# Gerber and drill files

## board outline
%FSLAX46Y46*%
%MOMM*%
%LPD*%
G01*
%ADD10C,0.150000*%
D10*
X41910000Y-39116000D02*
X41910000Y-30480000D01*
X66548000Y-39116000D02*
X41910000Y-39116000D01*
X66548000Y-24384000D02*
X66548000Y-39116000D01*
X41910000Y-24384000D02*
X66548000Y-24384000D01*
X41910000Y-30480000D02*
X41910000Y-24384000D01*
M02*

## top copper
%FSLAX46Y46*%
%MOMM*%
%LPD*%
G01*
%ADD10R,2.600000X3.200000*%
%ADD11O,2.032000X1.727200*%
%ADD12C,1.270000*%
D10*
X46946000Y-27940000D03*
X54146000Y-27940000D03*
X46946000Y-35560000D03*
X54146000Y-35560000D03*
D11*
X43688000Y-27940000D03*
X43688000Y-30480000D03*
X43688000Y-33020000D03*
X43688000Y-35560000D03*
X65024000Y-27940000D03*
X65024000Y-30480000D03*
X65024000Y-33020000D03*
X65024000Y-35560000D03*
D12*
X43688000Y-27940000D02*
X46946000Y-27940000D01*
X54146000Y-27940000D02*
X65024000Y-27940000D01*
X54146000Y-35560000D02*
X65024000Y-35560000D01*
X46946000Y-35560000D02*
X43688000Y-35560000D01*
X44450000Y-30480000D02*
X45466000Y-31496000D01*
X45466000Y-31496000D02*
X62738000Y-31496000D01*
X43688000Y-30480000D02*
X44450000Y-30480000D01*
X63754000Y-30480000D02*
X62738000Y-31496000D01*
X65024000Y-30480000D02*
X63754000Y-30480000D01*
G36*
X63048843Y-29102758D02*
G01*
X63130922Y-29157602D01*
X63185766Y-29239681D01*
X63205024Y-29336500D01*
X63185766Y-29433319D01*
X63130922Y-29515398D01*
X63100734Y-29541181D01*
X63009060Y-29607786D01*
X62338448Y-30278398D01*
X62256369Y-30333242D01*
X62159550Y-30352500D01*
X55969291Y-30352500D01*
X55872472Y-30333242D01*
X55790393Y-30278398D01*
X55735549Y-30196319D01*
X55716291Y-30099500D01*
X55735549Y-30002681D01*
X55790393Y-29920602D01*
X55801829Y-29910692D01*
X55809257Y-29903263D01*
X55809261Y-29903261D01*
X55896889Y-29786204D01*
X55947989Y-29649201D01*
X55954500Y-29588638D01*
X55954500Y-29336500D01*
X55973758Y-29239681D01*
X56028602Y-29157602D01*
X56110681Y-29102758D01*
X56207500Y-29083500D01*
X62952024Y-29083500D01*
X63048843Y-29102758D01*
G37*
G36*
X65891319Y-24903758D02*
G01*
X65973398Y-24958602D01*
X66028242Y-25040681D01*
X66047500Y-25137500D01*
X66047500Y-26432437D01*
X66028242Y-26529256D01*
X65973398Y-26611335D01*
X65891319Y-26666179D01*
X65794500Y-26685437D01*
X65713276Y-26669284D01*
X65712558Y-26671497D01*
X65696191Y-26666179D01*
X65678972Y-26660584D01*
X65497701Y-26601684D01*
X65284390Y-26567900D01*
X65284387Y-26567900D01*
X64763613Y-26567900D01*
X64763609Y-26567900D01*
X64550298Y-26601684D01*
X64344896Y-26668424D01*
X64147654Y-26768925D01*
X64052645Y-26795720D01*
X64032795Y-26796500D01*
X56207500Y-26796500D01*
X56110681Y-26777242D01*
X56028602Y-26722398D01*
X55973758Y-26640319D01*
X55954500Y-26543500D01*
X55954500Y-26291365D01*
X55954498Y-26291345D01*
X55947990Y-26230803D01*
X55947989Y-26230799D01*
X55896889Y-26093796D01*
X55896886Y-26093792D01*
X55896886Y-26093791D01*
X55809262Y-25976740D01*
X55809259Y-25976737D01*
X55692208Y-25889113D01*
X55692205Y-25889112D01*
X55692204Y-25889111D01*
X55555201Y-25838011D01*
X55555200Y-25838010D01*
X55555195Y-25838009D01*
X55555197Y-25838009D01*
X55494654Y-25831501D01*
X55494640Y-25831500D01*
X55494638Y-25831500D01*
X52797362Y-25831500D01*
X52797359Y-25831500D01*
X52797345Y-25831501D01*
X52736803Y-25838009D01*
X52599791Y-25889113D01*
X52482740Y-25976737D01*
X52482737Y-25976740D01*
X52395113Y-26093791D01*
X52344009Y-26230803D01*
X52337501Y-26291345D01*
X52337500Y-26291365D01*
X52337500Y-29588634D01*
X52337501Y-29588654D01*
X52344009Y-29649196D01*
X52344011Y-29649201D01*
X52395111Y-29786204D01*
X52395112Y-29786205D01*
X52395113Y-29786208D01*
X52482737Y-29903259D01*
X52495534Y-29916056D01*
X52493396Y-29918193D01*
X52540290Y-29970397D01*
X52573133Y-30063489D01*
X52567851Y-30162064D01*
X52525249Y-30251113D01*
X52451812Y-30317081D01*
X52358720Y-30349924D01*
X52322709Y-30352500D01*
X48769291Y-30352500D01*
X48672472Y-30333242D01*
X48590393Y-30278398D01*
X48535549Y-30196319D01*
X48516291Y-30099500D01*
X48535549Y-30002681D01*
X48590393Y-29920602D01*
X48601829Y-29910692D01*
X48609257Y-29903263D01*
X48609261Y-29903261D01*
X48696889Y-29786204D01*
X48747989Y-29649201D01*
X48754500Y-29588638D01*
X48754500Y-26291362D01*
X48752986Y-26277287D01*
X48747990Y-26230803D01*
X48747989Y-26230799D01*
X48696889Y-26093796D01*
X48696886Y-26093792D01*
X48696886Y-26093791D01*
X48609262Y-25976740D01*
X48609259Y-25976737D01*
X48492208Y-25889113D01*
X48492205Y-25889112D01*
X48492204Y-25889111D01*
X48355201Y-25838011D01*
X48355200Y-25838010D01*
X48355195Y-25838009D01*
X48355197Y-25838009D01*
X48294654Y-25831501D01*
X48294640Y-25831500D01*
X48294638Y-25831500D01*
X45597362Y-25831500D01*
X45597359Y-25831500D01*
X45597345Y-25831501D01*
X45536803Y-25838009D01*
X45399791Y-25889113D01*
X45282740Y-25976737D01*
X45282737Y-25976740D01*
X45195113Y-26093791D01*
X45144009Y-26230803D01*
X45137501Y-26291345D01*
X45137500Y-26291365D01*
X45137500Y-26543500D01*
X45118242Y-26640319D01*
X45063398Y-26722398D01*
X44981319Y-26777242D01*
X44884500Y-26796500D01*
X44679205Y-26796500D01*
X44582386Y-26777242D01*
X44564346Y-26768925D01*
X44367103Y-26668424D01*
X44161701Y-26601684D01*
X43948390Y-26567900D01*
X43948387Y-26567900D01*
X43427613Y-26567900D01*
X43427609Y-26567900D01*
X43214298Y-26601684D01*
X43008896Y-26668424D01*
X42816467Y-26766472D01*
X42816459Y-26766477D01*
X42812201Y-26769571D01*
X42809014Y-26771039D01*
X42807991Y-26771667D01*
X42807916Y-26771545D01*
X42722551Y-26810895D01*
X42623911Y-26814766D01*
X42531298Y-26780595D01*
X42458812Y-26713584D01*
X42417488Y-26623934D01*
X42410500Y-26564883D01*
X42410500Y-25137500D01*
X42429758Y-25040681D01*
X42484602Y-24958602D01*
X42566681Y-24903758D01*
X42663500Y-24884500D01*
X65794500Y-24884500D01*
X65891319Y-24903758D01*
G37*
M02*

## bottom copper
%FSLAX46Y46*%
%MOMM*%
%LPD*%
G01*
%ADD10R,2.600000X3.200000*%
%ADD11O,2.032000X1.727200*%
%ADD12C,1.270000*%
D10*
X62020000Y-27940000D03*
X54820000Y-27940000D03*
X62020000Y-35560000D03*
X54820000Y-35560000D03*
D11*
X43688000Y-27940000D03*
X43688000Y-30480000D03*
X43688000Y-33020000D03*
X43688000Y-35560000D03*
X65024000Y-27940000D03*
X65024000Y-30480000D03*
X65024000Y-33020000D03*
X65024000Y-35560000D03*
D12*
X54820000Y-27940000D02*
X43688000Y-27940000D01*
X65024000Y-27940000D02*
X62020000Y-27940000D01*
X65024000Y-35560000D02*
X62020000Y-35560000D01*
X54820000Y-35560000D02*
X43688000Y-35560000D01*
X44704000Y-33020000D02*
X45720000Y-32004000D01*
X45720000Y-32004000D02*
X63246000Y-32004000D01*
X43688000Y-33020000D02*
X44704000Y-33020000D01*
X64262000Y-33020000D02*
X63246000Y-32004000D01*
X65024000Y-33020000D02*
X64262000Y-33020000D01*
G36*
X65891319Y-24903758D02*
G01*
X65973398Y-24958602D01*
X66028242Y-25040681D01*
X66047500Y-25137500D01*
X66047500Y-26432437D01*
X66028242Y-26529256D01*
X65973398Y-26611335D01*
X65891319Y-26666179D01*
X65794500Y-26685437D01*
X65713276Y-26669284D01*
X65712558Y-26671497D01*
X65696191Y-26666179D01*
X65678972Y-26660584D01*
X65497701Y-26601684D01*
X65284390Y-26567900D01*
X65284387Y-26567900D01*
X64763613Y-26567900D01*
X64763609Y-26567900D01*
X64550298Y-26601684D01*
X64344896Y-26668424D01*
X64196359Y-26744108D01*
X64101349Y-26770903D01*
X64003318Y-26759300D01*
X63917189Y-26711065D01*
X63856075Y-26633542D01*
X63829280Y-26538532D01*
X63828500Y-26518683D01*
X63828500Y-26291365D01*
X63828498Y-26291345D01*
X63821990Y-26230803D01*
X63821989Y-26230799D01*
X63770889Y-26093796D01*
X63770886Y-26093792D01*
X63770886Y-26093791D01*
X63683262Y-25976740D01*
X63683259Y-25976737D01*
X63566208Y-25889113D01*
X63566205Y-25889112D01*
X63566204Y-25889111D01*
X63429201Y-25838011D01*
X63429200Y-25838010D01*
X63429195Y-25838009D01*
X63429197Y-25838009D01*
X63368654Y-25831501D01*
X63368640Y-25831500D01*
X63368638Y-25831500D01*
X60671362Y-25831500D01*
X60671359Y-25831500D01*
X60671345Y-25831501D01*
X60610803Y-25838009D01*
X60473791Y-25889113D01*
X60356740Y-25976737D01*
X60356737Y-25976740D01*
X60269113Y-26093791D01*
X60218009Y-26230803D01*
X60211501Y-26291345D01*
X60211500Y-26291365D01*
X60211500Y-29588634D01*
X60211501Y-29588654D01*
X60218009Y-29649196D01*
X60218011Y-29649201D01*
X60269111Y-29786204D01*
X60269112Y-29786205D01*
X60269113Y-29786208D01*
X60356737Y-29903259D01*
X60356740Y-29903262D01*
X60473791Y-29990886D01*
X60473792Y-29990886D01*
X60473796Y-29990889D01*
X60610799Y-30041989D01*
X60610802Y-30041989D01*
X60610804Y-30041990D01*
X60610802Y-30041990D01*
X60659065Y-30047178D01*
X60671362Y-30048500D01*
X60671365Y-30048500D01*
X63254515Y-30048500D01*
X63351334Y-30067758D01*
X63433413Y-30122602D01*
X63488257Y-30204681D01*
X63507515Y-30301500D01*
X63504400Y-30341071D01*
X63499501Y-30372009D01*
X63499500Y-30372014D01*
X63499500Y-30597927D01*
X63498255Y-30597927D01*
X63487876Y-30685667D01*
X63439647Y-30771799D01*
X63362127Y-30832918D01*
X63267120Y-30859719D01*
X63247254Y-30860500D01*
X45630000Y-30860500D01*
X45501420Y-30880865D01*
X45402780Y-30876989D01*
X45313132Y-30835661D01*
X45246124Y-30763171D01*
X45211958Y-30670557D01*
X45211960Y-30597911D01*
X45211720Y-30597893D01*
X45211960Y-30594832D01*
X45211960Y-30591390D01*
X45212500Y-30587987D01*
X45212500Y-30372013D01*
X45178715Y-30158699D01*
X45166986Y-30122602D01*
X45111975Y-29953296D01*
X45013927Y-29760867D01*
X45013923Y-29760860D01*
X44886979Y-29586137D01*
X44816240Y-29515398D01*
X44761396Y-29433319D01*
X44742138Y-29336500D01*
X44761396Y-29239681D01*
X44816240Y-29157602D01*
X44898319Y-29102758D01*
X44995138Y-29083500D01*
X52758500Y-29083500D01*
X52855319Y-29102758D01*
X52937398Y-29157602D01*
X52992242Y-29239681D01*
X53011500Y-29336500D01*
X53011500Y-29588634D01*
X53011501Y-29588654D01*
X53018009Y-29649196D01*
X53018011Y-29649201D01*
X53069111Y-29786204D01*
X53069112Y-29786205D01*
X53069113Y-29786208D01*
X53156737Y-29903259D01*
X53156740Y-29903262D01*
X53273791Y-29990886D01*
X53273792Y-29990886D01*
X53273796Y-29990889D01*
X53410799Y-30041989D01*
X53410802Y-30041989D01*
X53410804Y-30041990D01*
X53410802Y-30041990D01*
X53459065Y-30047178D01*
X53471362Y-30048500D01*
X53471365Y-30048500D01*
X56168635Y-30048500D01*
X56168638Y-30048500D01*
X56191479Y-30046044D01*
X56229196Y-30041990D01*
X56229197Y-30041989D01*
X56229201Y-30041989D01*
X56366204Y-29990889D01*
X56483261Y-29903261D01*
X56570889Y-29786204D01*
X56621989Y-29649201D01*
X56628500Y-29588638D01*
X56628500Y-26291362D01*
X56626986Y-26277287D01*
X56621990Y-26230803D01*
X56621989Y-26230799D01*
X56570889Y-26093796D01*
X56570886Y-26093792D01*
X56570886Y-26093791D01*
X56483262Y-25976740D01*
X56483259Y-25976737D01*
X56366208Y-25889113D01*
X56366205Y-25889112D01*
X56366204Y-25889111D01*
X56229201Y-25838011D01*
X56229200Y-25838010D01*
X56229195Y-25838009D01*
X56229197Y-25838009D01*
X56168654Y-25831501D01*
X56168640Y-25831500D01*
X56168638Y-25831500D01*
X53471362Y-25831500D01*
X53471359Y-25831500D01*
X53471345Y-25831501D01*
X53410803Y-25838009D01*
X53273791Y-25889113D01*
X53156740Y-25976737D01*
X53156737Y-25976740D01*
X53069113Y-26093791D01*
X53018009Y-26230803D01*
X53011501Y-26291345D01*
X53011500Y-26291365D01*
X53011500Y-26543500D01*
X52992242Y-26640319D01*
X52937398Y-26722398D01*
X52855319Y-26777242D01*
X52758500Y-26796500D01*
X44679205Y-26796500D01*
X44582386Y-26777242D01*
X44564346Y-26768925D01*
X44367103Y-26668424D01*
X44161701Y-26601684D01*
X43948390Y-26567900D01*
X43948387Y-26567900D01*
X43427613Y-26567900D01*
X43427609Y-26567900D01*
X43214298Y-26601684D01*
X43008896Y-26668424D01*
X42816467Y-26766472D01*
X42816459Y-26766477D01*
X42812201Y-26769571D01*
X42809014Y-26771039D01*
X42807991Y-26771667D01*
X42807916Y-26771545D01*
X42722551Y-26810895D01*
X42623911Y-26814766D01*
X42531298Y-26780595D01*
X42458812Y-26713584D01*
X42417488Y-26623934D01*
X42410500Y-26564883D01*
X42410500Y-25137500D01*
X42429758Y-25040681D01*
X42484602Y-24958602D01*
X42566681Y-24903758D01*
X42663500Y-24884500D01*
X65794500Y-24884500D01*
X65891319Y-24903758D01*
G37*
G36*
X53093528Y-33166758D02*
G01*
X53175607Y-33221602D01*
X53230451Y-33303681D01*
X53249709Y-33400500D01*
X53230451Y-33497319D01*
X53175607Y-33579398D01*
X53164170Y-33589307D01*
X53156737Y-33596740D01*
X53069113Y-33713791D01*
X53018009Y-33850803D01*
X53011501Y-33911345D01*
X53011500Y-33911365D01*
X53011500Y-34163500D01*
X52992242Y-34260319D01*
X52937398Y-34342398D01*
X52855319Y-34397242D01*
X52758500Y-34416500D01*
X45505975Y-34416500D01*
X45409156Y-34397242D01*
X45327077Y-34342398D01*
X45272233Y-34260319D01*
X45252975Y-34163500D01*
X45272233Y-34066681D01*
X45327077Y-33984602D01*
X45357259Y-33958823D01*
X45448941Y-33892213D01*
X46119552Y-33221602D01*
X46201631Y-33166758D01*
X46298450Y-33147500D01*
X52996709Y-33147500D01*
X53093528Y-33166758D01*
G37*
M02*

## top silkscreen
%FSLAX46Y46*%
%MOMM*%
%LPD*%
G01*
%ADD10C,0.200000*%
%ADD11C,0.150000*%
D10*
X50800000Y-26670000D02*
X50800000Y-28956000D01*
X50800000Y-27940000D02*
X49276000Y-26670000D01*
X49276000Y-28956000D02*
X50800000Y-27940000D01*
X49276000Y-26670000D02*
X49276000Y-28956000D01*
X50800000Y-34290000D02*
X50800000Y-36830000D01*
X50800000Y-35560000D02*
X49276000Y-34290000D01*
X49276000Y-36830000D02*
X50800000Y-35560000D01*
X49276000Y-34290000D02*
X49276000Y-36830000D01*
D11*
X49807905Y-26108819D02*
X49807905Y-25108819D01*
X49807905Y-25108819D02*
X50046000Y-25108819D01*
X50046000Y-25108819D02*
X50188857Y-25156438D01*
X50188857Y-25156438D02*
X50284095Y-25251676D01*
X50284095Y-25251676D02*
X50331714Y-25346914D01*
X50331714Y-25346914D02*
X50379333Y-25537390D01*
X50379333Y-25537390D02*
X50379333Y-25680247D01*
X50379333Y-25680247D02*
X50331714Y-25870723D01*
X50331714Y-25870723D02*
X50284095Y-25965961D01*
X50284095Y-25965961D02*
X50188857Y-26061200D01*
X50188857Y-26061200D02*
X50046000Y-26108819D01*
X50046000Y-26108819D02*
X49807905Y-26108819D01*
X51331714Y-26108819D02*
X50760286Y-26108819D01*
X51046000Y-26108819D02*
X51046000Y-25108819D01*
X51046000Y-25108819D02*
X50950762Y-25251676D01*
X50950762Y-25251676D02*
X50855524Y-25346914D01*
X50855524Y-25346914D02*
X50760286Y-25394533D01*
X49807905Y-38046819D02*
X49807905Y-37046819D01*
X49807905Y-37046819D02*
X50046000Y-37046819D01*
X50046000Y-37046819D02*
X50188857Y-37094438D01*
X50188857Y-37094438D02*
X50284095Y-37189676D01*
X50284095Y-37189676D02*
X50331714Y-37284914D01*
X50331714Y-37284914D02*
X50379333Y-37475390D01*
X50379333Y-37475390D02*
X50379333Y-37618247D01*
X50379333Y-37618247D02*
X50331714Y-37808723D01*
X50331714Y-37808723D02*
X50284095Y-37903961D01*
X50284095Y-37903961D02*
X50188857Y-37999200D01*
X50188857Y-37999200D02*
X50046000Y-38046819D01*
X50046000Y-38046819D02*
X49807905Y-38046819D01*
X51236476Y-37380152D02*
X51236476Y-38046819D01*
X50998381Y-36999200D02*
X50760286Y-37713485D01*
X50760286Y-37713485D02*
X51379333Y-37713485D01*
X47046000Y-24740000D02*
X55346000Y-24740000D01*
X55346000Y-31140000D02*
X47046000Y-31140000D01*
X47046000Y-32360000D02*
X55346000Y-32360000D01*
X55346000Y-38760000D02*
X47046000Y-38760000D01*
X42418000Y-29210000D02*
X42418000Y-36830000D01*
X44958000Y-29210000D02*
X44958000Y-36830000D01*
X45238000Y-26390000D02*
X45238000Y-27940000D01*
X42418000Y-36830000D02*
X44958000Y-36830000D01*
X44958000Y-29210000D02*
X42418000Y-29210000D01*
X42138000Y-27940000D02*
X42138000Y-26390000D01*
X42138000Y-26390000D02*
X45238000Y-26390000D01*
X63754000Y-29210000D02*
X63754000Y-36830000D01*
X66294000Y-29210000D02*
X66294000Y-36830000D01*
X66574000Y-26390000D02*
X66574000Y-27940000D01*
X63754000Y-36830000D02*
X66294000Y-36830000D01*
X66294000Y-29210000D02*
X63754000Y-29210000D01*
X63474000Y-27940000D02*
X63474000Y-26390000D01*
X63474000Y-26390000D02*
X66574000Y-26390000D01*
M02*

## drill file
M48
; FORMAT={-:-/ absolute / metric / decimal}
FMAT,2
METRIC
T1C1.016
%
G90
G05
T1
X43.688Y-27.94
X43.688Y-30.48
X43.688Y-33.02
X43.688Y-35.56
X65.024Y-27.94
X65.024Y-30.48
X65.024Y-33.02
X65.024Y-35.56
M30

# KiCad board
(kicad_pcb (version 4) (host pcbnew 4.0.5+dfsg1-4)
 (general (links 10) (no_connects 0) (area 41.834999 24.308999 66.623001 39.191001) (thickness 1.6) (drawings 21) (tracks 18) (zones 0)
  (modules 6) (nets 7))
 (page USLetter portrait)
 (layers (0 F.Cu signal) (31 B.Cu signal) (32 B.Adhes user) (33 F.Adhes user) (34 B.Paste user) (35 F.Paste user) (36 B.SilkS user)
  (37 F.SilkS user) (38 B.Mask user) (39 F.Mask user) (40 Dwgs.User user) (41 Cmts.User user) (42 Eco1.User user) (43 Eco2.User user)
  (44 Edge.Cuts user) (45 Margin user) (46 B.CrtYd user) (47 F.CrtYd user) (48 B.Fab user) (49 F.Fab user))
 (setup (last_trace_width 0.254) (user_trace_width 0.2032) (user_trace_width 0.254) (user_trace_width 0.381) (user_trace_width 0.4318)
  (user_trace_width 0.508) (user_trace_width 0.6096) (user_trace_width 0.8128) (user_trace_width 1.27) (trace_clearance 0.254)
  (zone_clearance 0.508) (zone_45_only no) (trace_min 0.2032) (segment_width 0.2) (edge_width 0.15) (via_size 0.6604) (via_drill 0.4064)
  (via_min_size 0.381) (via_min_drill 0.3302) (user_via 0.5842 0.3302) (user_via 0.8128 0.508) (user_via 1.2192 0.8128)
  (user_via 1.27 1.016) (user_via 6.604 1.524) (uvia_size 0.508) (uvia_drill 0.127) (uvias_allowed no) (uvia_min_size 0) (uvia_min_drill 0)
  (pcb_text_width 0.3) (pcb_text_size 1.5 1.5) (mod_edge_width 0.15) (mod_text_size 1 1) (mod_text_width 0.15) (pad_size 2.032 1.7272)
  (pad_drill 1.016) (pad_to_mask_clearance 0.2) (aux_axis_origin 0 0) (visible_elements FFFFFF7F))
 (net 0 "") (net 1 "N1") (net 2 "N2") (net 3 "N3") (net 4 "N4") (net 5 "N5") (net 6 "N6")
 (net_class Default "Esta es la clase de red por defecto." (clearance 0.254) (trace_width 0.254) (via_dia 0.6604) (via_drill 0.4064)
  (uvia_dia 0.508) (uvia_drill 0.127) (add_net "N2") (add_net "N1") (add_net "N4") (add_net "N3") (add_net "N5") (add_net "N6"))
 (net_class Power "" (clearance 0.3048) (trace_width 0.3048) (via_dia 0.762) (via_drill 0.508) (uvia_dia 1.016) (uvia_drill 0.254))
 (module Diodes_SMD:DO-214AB (layer F.Cu) (at 50.546 27.94 180)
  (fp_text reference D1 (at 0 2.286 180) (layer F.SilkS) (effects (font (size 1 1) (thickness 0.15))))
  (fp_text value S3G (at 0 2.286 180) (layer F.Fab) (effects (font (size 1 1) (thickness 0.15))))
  (fp_line (start 3.5 3.2) (end -4.8 3.2) (layer F.SilkS) (width 0.15))
  (fp_line (start -4.8 -3.2) (end 3.5 -3.2) (layer F.SilkS) (width 0.15))
  (pad 2 smd rect (at 3.6 0 180) (size 2.6 3.2) (layers F.Cu F.Paste F.Mask) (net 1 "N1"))
  (pad 1 smd rect (at -3.6 0 180) (size 2.6 3.2) (layers F.Cu F.Paste F.Mask) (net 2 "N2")))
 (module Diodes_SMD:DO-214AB (layer B.Cu) (at 58.42 27.94)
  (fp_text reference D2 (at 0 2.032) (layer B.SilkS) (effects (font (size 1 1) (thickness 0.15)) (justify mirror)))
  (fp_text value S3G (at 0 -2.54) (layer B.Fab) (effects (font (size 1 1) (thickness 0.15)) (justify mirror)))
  (pad 2 smd rect (at 3.6 0) (size 2.6 3.2) (layers B.Cu B.Paste B.Mask) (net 2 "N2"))
  (pad 1 smd rect (at -3.6 0) (size 2.6 3.2) (layers B.Cu B.Paste B.Mask) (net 1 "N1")))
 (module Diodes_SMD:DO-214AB (layer B.Cu) (at 58.42 35.56)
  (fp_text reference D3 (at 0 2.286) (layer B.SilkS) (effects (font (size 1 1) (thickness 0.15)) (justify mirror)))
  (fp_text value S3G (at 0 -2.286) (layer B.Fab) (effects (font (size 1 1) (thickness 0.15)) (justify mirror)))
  (pad 2 smd rect (at 3.6 0) (size 2.6 3.2) (layers B.Cu B.Paste B.Mask) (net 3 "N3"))
  (pad 1 smd rect (at -3.6 0) (size 2.6 3.2) (layers B.Cu B.Paste B.Mask) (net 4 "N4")))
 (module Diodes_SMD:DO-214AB (layer F.Cu) (at 50.546 35.56 180)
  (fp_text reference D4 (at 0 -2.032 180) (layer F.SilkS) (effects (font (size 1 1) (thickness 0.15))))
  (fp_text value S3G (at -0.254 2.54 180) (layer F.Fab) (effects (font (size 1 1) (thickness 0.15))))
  (fp_line (start 3.5 3.2) (end -4.8 3.2) (layer F.SilkS) (width 0.15))
  (fp_line (start -4.8 -3.2) (end 3.5 -3.2) (layer F.SilkS) (width 0.15))
  (pad 2 smd rect (at 3.6 0 180) (size 2.6 3.2) (layers F.Cu F.Paste F.Mask) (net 4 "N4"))
  (pad 1 smd rect (at -3.6 0 180) (size 2.6 3.2) (layers F.Cu F.Paste F.Mask) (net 3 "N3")))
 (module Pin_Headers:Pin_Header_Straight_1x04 (layer F.Cu) (at 43.688 27.94)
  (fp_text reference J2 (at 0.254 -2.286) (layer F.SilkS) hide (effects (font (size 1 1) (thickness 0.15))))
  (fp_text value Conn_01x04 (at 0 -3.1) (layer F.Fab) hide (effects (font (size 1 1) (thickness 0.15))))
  (fp_line (start -1.27 1.27) (end -1.27 8.89) (layer F.SilkS) (width 0.15))
  (fp_line (start 1.27 1.27) (end 1.27 8.89) (layer F.SilkS) (width 0.15))
  (fp_line (start 1.55 -1.55) (end 1.55 0) (layer F.SilkS) (width 0.15))
  (fp_line (start -1.27 8.89) (end 1.27 8.89) (layer F.SilkS) (width 0.15))
  (fp_line (start 1.27 1.27) (end -1.27 1.27) (layer F.SilkS) (width 0.15))
  (fp_line (start -1.55 0) (end -1.55 -1.55) (layer F.SilkS) (width 0.15))
  (fp_line (start -1.55 -1.55) (end 1.55 -1.55) (layer F.SilkS) (width 0.15))
  (pad 1 thru_hole oval (at 0 0) (size 2.032 1.7272) (drill 1.016) (layers *.Cu *.Mask) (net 1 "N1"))
  (pad 2 thru_hole oval (at 0 2.54) (size 2.032 1.7272) (drill 1.016) (layers *.Cu *.Mask) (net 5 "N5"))
  (pad 3 thru_hole oval (at 0 5.08) (size 2.032 1.7272) (drill 1.016) (layers *.Cu *.Mask) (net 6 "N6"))
  (pad 4 thru_hole oval (at 0 7.62) (size 2.032 1.7272) (drill 1.016) (layers *.Cu *.Mask) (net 4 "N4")))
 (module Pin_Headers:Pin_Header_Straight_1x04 (layer F.Cu) (at 65.024 27.94)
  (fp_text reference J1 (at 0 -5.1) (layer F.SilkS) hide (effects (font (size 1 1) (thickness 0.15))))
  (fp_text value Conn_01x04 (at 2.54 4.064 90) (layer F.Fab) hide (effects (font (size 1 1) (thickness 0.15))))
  (fp_line (start -1.27 1.27) (end -1.27 8.89) (layer F.SilkS) (width 0.15))
  (fp_line (start 1.27 1.27) (end 1.27 8.89) (layer F.SilkS) (width 0.15))
  (fp_line (start 1.55 -1.55) (end 1.55 0) (layer F.SilkS) (width 0.15))
  (fp_line (start -1.27 8.89) (end 1.27 8.89) (layer F.SilkS) (width 0.15))
  (fp_line (start 1.27 1.27) (end -1.27 1.27) (layer F.SilkS) (width 0.15))
  (fp_line (start -1.55 0) (end -1.55 -1.55) (layer F.SilkS) (width 0.15))
  (fp_line (start -1.55 -1.55) (end 1.55 -1.55) (layer F.SilkS) (width 0.15))
  (pad 1 thru_hole oval (at 0 0) (size 2.032 1.7272) (drill 1.016) (layers *.Cu *.Mask) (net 2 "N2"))
  (pad 2 thru_hole oval (at 0 2.54) (size 2.032 1.7272) (drill 1.016) (layers *.Cu *.Mask) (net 5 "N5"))
  (pad 3 thru_hole oval (at 0 5.08) (size 2.032 1.7272) (drill 1.016) (layers *.Cu *.Mask) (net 6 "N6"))
  (pad 4 thru_hole oval (at 0 7.62) (size 2.032 1.7272) (drill 1.016) (layers *.Cu *.Mask) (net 3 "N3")))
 (gr_line (start 50.8 26.67) (end 50.8 28.956) (layer F.SilkS) (width 0.2))
 (gr_line (start 50.8 27.94) (end 49.276 26.67) (layer F.SilkS) (width 0.2))
 (gr_line (start 49.276 28.956) (end 50.8 27.94) (layer F.SilkS) (width 0.2))
 (gr_line (start 49.276 26.67) (end 49.276 28.956) (layer F.SilkS) (width 0.2))
 (gr_line (start 50.8 34.29) (end 50.8 36.83) (layer F.SilkS) (width 0.2))
 (gr_line (start 50.8 35.56) (end 49.276 34.29) (layer F.SilkS) (width 0.2))
 (gr_line (start 49.276 36.83) (end 50.8 35.56) (layer F.SilkS) (width 0.2))
 (gr_line (start 49.276 34.29) (end 49.276 36.83) (layer F.SilkS) (width 0.2))
 (gr_line (start 41.91 39.116) (end 41.91 30.48) (layer Edge.Cuts) (width 0.15))
 (gr_line (start 66.548 39.116) (end 41.91 39.116) (layer Edge.Cuts) (width 0.15))
 (gr_line (start 66.548 24.384) (end 66.548 39.116) (layer Edge.Cuts) (width 0.15))
 (gr_line (start 41.91 24.384) (end 66.548 24.384) (layer Edge.Cuts) (width 0.15))
 (gr_line (start 41.91 30.48) (end 41.91 24.384) (layer Edge.Cuts) (width 0.15))
 (segment (start 43.688 27.94) (end 46.946 27.94) (width 1.27) (layer F.Cu) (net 1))
 (segment (start 54.82 27.94) (end 43.688 27.94) (width 1.27) (layer B.Cu) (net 1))
 (segment (start 54.146 27.94) (end 65.024 27.94) (width 1.27) (layer F.Cu) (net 2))
 (segment (start 65.024 27.94) (end 62.02 27.94) (width 1.27) (layer B.Cu) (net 2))
 (segment (start 54.146 35.56) (end 65.024 35.56) (width 1.27) (layer F.Cu) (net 3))
 (segment (start 65.024 35.56) (end 62.02 35.56) (width 1.27) (layer B.Cu) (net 3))
 (segment (start 46.946 35.56) (end 43.688 35.56) (width 1.27) (layer F.Cu) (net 4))
 (segment (start 54.82 35.56) (end 43.688 35.56) (width 1.27) (layer B.Cu) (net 4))
 (segment (start 44.45 30.48) (end 45.466 31.496) (width 1.27) (layer F.Cu) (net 5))
 (segment (start 45.466 31.496) (end 62.738 31.496) (width 1.27) (layer F.Cu) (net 5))
 (segment (start 43.688 30.48) (end 44.45 30.48) (width 1.27) (layer F.Cu) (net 5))
 (segment (start 63.754 30.48) (end 62.738 31.496) (width 1.27) (layer F.Cu) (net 5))
 (segment (start 65.024 30.48) (end 63.754 30.48) (width 1.27) (layer F.Cu) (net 5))
 (segment (start 44.704 33.02) (end 45.72 32.004) (width 1.27) (layer B.Cu) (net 6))
 (segment (start 45.72 32.004) (end 63.246 32.004) (width 1.27) (layer B.Cu) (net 6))
 (segment (start 43.688 33.02) (end 44.704 33.02) (width 1.27) (layer B.Cu) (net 6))
 (segment (start 64.262 33.02) (end 63.246 32.004) (width 1.27) (layer B.Cu) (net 6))
 (segment (start 65.024 33.02) (end 64.262 33.02) (width 1.27) (layer B.Cu) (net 6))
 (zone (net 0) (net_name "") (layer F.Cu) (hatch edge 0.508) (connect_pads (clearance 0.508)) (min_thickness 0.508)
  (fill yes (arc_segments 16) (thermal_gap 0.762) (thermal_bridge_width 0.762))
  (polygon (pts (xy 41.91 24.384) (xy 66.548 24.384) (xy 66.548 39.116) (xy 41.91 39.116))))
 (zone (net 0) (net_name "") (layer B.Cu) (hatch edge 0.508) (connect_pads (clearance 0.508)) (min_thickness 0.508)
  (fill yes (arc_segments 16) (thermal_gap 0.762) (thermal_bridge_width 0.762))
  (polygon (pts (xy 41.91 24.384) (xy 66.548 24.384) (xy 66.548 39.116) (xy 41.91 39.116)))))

